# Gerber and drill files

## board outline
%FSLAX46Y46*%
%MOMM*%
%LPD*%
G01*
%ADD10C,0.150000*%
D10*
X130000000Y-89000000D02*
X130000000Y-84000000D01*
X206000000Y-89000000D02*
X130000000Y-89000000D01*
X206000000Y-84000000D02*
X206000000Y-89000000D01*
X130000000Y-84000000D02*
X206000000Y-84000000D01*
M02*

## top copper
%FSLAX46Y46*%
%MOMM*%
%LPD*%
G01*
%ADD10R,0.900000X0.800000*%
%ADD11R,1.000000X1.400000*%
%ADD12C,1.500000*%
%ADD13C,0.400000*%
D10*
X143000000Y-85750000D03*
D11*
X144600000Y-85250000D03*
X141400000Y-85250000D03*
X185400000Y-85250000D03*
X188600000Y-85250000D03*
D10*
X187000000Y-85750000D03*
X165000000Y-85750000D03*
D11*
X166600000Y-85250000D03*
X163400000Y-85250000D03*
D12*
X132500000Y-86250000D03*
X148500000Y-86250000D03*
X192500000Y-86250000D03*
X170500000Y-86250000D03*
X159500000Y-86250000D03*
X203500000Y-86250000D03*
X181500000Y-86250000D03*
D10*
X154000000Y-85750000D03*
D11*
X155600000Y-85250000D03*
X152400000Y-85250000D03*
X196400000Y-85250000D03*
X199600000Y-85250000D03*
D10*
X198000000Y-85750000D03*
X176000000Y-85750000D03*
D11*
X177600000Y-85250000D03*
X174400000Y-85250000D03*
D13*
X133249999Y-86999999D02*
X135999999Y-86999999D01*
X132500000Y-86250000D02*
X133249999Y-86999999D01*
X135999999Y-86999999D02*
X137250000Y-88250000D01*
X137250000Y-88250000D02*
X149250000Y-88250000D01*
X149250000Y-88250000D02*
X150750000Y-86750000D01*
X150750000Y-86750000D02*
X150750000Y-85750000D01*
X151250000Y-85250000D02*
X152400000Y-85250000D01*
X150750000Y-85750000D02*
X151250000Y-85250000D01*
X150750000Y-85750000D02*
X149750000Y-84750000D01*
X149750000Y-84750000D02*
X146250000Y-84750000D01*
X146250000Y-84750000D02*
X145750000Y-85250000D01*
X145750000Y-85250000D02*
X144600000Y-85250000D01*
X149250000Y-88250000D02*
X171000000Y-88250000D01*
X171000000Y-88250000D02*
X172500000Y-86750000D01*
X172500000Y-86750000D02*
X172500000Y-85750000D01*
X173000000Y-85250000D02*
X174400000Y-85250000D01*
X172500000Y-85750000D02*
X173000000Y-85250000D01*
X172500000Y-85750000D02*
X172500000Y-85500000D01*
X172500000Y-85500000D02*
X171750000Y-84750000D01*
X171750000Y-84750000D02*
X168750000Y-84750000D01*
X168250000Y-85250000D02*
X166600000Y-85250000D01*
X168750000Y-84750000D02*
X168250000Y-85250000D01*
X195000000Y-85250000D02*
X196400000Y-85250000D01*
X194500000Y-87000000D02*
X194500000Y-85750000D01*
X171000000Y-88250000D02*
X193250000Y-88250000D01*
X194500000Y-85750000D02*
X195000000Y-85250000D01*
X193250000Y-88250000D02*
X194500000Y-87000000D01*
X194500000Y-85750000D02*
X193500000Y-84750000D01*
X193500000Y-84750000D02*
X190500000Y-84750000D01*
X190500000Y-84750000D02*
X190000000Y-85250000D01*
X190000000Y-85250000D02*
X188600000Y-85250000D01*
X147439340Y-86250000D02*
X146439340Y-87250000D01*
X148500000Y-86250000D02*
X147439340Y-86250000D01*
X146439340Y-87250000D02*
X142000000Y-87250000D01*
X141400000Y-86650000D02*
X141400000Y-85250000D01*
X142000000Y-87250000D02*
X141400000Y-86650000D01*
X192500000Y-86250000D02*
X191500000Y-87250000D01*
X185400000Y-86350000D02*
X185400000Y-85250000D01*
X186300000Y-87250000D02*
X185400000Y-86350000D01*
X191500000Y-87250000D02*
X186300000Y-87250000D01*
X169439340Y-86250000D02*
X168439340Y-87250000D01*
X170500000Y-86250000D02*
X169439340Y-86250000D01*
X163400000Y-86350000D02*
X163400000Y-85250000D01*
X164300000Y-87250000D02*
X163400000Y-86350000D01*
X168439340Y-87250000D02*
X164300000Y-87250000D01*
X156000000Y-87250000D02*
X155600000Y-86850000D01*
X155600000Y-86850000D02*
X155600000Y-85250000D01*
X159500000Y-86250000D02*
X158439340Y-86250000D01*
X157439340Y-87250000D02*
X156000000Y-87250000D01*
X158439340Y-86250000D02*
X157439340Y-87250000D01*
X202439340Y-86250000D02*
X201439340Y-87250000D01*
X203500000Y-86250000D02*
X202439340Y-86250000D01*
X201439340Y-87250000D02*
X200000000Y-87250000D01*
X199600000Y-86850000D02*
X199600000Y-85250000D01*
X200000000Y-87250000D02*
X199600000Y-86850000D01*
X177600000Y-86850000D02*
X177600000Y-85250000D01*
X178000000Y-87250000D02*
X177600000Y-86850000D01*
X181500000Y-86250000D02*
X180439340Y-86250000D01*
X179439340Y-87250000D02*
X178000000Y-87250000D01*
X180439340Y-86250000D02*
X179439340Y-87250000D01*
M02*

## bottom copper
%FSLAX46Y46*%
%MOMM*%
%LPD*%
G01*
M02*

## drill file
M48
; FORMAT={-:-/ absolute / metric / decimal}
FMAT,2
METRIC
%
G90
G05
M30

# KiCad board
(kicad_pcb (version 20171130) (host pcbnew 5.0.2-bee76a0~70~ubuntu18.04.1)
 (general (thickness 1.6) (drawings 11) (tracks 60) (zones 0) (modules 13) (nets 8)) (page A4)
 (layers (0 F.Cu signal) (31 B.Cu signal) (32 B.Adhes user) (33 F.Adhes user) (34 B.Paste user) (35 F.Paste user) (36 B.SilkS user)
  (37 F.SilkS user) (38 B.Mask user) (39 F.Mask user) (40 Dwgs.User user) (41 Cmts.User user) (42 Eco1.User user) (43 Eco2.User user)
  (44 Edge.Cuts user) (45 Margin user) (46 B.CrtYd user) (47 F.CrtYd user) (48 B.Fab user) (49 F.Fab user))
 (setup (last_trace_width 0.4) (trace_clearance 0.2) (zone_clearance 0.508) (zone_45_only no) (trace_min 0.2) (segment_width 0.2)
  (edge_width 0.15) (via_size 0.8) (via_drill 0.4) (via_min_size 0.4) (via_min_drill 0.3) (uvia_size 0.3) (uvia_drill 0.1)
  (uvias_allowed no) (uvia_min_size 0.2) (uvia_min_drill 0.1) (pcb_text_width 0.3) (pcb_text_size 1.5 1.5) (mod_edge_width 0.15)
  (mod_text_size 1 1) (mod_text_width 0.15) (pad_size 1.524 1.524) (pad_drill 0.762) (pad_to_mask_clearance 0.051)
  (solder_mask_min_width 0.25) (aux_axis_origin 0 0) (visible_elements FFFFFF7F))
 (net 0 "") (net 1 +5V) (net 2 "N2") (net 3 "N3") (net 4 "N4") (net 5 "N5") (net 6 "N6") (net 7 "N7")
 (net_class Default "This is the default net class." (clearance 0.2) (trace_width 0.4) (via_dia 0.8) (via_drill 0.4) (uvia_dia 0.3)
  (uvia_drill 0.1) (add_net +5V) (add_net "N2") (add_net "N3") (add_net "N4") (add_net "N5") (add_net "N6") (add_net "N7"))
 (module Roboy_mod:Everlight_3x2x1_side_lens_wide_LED (layer F.Cu) (at 143 85.25)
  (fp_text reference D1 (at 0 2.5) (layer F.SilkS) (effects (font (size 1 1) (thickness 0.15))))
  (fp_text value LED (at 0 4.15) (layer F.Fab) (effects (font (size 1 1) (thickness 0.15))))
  (pad "" smd rect (at 0 0.5) (size 0.9 0.8) (layers F.Cu F.Paste F.Mask))
  (pad 2 smd rect (at 1.6 0) (size 1 1.4) (layers F.Cu F.Paste F.Mask) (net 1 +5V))
  (pad 1 smd rect (at -1.6 0) (size 1 1.4) (layers F.Cu F.Paste F.Mask) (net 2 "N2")))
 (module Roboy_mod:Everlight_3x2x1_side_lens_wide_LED (layer F.Cu) (at 187 85.25)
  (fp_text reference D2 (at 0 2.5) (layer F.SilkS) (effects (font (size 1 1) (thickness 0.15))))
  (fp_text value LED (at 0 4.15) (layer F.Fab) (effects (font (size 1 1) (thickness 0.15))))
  (pad 1 smd rect (at -1.6 0) (size 1 1.4) (layers F.Cu F.Paste F.Mask) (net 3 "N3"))
  (pad 2 smd rect (at 1.6 0) (size 1 1.4) (layers F.Cu F.Paste F.Mask) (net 1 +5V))
  (pad "" smd rect (at 0 0.5) (size 0.9 0.8) (layers F.Cu F.Paste F.Mask)))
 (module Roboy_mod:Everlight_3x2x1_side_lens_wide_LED (layer F.Cu) (at 165 85.25)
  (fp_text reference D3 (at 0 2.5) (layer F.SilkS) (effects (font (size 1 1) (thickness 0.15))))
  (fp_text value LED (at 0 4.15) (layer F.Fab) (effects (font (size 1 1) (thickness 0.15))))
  (pad "" smd rect (at 0 0.5) (size 0.9 0.8) (layers F.Cu F.Paste F.Mask))
  (pad 2 smd rect (at 1.6 0) (size 1 1.4) (layers F.Cu F.Paste F.Mask) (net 1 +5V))
  (pad 1 smd rect (at -1.6 0) (size 1 1.4) (layers F.Cu F.Paste F.Mask) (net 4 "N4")))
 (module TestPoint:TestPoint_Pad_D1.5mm (layer F.Cu) (at 132.5 86.25)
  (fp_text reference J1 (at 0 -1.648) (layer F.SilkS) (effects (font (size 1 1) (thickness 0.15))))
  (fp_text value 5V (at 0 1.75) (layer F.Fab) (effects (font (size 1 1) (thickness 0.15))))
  (pad 1 smd circle (at 0 0) (size 1.5 1.5) (layers F.Cu F.Mask) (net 1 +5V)))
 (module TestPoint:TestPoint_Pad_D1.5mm (layer F.Cu) (at 148.5 86.25)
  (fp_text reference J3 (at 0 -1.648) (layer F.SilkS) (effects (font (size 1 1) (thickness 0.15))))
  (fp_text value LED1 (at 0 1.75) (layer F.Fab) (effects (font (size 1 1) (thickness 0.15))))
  (pad 1 smd circle (at 0 0) (size 1.5 1.5) (layers F.Cu F.Mask) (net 2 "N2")))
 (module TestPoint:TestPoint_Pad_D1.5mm (layer F.Cu) (at 192.5 86.25)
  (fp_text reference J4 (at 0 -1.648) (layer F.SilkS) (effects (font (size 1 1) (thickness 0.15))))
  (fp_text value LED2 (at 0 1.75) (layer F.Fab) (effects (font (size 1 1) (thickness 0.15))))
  (pad 1 smd circle (at 0 0) (size 1.5 1.5) (layers F.Cu F.Mask) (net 3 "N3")))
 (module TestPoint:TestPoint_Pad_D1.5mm (layer F.Cu) (at 170.5 86.25)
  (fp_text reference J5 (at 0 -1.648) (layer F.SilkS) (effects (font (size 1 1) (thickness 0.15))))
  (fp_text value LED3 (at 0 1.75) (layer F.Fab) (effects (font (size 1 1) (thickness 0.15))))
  (pad 1 smd circle (at 0 0) (size 1.5 1.5) (layers F.Cu F.Mask) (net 4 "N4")))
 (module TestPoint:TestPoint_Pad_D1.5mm (layer F.Cu) (at 159.5 86.25)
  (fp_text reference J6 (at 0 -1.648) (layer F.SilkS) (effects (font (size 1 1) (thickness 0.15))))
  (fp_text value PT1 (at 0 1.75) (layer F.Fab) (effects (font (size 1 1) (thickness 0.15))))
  (pad 1 smd circle (at 0 0) (size 1.5 1.5) (layers F.Cu F.Mask) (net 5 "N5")))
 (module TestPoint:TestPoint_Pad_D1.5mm (layer F.Cu) (at 203.5 86.25)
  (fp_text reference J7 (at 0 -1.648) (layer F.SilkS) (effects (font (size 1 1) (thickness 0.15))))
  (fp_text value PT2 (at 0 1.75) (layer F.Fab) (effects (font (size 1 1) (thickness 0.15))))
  (pad 1 smd circle (at 0 0) (size 1.5 1.5) (layers F.Cu F.Mask) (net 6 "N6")))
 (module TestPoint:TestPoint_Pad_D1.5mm (layer F.Cu) (at 181.5 86.25)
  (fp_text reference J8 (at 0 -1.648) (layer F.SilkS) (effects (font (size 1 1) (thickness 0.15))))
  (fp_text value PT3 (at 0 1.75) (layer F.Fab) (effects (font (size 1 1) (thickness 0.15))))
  (pad 1 smd circle (at 0 0) (size 1.5 1.5) (layers F.Cu F.Mask) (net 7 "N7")))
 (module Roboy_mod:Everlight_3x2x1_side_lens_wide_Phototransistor (layer F.Cu) (at 154 85.25)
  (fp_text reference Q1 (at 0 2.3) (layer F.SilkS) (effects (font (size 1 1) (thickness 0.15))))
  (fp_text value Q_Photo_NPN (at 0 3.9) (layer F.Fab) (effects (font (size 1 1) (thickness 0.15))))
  (pad "" smd rect (at 0 0.5) (size 0.9 0.8) (layers F.Cu F.Paste F.Mask))
  (pad 2 smd rect (at 1.6 0) (size 1 1.4) (layers F.Cu F.Paste F.Mask) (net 5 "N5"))
  (pad 1 smd rect (at -1.6 0) (size 1 1.4) (layers F.Cu F.Paste F.Mask) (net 1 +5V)))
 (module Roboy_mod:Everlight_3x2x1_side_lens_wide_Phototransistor (layer F.Cu) (at 198 85.25)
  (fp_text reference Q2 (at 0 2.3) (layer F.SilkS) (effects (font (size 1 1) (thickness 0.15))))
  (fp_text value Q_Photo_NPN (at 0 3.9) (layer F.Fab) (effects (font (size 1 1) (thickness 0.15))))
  (pad 1 smd rect (at -1.6 0) (size 1 1.4) (layers F.Cu F.Paste F.Mask) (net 1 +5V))
  (pad 2 smd rect (at 1.6 0) (size 1 1.4) (layers F.Cu F.Paste F.Mask) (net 6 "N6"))
  (pad "" smd rect (at 0 0.5) (size 0.9 0.8) (layers F.Cu F.Paste F.Mask)))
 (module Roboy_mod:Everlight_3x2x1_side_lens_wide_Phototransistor (layer F.Cu) (at 176 85.25)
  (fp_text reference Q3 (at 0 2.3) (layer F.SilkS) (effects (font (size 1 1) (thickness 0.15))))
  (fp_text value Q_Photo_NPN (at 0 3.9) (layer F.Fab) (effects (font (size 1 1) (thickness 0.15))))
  (pad "" smd rect (at 0 0.5) (size 0.9 0.8) (layers F.Cu F.Paste F.Mask))
  (pad 2 smd rect (at 1.6 0) (size 1 1.4) (layers F.Cu F.Paste F.Mask) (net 7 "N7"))
  (pad 1 smd rect (at -1.6 0) (size 1 1.4) (layers F.Cu F.Paste F.Mask) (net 1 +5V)))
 (gr_line (start 130 89) (end 130 84) (layer Edge.Cuts) (width 0.15))
 (gr_line (start 206 89) (end 130 89) (layer Edge.Cuts) (width 0.15))
 (gr_line (start 206 84) (end 206 89) (layer Edge.Cuts) (width 0.15))
 (gr_line (start 130 84) (end 206 84) (layer Edge.Cuts) (width 0.15))
 (segment (start 133.249999 86.999999) (end 135.999999 86.999999) (width 0.4) (layer F.Cu) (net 1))
 (segment (start 132.5 86.25) (end 133.249999 86.999999) (width 0.4) (layer F.Cu) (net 1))
 (segment (start 135.999999 86.999999) (end 137.25 88.25) (width 0.4) (layer F.Cu) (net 1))
 (segment (start 137.25 88.25) (end 149.25 88.25) (width 0.4) (layer F.Cu) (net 1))
 (segment (start 149.25 88.25) (end 150.75 86.75) (width 0.4) (layer F.Cu) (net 1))
 (segment (start 150.75 86.75) (end 150.75 85.75) (width 0.4) (layer F.Cu) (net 1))
 (segment (start 151.25 85.25) (end 152.4 85.25) (width 0.4) (layer F.Cu) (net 1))
 (segment (start 150.75 85.75) (end 151.25 85.25) (width 0.4) (layer F.Cu) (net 1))
 (segment (start 150.75 85.75) (end 149.75 84.75) (width 0.4) (layer F.Cu) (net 1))
 (segment (start 149.75 84.75) (end 146.25 84.75) (width 0.4) (layer F.Cu) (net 1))
 (segment (start 146.25 84.75) (end 145.75 85.25) (width 0.4) (layer F.Cu) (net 1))
 (segment (start 145.75 85.25) (end 144.6 85.25) (width 0.4) (layer F.Cu) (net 1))
 (segment (start 149.25 88.25) (end 171 88.25) (width 0.4) (layer F.Cu) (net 1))
 (segment (start 171 88.25) (end 172.5 86.75) (width 0.4) (layer F.Cu) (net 1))
 (segment (start 172.5 86.75) (end 172.5 85.75) (width 0.4) (layer F.Cu) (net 1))
 (segment (start 173 85.25) (end 174.4 85.25) (width 0.4) (layer F.Cu) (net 1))
 (segment (start 172.5 85.75) (end 173 85.25) (width 0.4) (layer F.Cu) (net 1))
 (segment (start 172.5 85.75) (end 172.5 85.5) (width 0.4) (layer F.Cu) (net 1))
 (segment (start 172.5 85.5) (end 171.75 84.75) (width 0.4) (layer F.Cu) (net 1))
 (segment (start 171.75 84.75) (end 168.75 84.75) (width 0.4) (layer F.Cu) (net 1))
 (segment (start 168.25 85.25) (end 166.6 85.25) (width 0.4) (layer F.Cu) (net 1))
 (segment (start 168.75 84.75) (end 168.25 85.25) (width 0.4) (layer F.Cu) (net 1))
 (segment (start 195 85.25) (end 196.4 85.25) (width 0.4) (layer F.Cu) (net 1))
 (segment (start 194.5 87) (end 194.5 85.75) (width 0.4) (layer F.Cu) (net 1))
 (segment (start 171 88.25) (end 193.25 88.25) (width 0.4) (layer F.Cu) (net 1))
 (segment (start 194.5 85.75) (end 195 85.25) (width 0.4) (layer F.Cu) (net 1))
 (segment (start 193.25 88.25) (end 194.5 87) (width 0.4) (layer F.Cu) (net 1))
 (segment (start 194.5 85.75) (end 193.5 84.75) (width 0.4) (layer F.Cu) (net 1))
 (segment (start 193.5 84.75) (end 190.5 84.75) (width 0.4) (layer F.Cu) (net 1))
 (segment (start 190.5 84.75) (end 190 85.25) (width 0.4) (layer F.Cu) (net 1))
 (segment (start 190 85.25) (end 188.6 85.25) (width 0.4) (layer F.Cu) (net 1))
 (segment (start 147.43934 86.25) (end 146.43934 87.25) (width 0.4) (layer F.Cu) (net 2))
 (segment (start 148.5 86.25) (end 147.43934 86.25) (width 0.4) (layer F.Cu) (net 2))
 (segment (start 146.43934 87.25) (end 142 87.25) (width 0.4) (layer F.Cu) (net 2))
 (segment (start 141.4 86.65) (end 141.4 85.25) (width 0.4) (layer F.Cu) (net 2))
 (segment (start 142 87.25) (end 141.4 86.65) (width 0.4) (layer F.Cu) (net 2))
 (segment (start 192.5 86.25) (end 191.5 87.25) (width 0.4) (layer F.Cu) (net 3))
 (segment (start 185.4 86.35) (end 185.4 85.25) (width 0.4) (layer F.Cu) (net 3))
 (segment (start 186.3 87.25) (end 185.4 86.35) (width 0.4) (layer F.Cu) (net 3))
 (segment (start 191.5 87.25) (end 186.3 87.25) (width 0.4) (layer F.Cu) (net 3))
 (segment (start 169.43934 86.25) (end 168.43934 87.25) (width 0.4) (layer F.Cu) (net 4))
 (segment (start 170.5 86.25) (end 169.43934 86.25) (width 0.4) (layer F.Cu) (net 4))
 (segment (start 163.4 86.35) (end 163.4 85.25) (width 0.4) (layer F.Cu) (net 4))
 (segment (start 164.3 87.25) (end 163.4 86.35) (width 0.4) (layer F.Cu) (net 4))
 (segment (start 168.43934 87.25) (end 164.3 87.25) (width 0.4) (layer F.Cu) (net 4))
 (segment (start 156 87.25) (end 155.6 86.85) (width 0.4) (layer F.Cu) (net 5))
 (segment (start 155.6 86.85) (end 155.6 85.25) (width 0.4) (layer F.Cu) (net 5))
 (segment (start 159.5 86.25) (end 158.43934 86.25) (width 0.4) (layer F.Cu) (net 5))
 (segment (start 157.43934 87.25) (end 156 87.25) (width 0.4) (layer F.Cu) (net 5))
 (segment (start 158.43934 86.25) (end 157.43934 87.25) (width 0.4) (layer F.Cu) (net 5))
 (segment (start 202.43934 86.25) (end 201.43934 87.25) (width 0.4) (layer F.Cu) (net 6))
 (segment (start 203.5 86.25) (end 202.43934 86.25) (width 0.4) (layer F.Cu) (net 6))
 (segment (start 201.43934 87.25) (end 200 87.25) (width 0.4) (layer F.Cu) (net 6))
 (segment (start 199.6 86.85) (end 199.6 85.25) (width 0.4) (layer F.Cu) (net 6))
 (segment (start 200 87.25) (end 199.6 86.85) (width 0.4) (layer F.Cu) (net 6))
 (segment (start 177.6 86.85) (end 177.6 85.25) (width 0.4) (layer F.Cu) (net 7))
 (segment (start 178 87.25) (end 177.6 86.85) (width 0.4) (layer F.Cu) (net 7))
 (segment (start 181.5 86.25) (end 180.43934 86.25) (width 0.4) (layer F.Cu) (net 7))
 (segment (start 179.43934 87.25) (end 178 87.25) (width 0.4) (layer F.Cu) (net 7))
 (segment (start 180.43934 86.25) (end 179.43934 87.25) (width 0.4) (layer F.Cu) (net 7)))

